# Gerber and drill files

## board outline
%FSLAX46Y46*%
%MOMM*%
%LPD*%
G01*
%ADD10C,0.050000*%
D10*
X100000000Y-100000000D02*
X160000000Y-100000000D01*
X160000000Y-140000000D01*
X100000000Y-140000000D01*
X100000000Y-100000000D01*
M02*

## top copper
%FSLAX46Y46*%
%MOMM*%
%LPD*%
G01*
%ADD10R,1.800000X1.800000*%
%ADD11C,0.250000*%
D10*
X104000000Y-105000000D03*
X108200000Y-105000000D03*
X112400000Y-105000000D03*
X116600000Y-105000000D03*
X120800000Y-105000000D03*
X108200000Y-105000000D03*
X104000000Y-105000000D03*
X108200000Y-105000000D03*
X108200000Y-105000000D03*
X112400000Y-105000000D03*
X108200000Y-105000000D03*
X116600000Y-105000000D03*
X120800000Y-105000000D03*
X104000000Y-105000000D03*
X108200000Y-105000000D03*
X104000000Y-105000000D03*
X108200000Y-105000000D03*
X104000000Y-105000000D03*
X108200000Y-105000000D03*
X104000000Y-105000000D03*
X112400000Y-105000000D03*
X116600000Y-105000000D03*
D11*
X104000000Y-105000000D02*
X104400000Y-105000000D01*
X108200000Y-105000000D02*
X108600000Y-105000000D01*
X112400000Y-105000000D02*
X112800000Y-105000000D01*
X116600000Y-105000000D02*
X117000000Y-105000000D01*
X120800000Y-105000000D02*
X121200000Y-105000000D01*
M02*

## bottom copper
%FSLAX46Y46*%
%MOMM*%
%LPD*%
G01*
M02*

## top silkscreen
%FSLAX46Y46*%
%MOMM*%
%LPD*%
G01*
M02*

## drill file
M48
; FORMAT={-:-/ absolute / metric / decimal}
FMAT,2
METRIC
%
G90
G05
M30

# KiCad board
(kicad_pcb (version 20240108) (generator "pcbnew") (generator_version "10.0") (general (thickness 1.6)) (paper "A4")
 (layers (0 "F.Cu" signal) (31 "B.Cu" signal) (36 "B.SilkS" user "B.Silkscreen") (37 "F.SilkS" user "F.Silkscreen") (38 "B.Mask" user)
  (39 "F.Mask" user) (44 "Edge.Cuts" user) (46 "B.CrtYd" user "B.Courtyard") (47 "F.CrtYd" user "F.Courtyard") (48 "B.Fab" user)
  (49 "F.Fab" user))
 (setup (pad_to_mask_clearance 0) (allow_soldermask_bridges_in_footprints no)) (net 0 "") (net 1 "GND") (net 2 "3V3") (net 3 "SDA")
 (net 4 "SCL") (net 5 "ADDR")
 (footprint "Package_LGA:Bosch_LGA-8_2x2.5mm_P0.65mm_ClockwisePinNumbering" (layer "F.Cu") (at 100 100)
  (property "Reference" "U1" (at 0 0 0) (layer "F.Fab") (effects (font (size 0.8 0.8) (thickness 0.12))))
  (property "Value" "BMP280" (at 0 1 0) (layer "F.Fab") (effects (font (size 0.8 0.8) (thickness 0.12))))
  (pad "1" smd rect (at 4.000 5.000) (size 1.8 1.8) (layers "F.Cu" "F.Paste" "F.Mask") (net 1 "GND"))
  (pad "2" smd rect (at 8.200 5.000) (size 1.8 1.8) (layers "F.Cu" "F.Paste" "F.Mask") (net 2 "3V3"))
  (pad "3" smd rect (at 12.400 5.000) (size 1.8 1.8) (layers "F.Cu" "F.Paste" "F.Mask") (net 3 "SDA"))
  (pad "4" smd rect (at 16.600 5.000) (size 1.8 1.8) (layers "F.Cu" "F.Paste" "F.Mask") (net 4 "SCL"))
  (pad "5" smd rect (at 20.800 5.000) (size 1.8 1.8) (layers "F.Cu" "F.Paste" "F.Mask") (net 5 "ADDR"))
  (pad "6" smd rect (at 8.200 5.000) (size 1.8 1.8) (layers "F.Cu" "F.Paste" "F.Mask") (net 2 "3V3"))
  (pad "7" smd rect (at 4.000 5.000) (size 1.8 1.8) (layers "F.Cu" "F.Paste" "F.Mask") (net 1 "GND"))
  (pad "8" smd rect (at 8.200 5.000) (size 1.8 1.8) (layers "F.Cu" "F.Paste" "F.Mask") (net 2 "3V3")))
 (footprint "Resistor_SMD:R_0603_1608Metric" (layer "F.Cu") (at 100 100)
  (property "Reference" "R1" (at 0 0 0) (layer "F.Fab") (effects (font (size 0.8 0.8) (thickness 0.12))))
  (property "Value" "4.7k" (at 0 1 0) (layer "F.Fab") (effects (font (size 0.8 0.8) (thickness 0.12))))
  (pad "1" smd rect (at 8.200 5.000) (size 1.8 1.8) (layers "F.Cu" "F.Paste" "F.Mask") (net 2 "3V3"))
  (pad "2" smd rect (at 12.400 5.000) (size 1.8 1.8) (layers "F.Cu" "F.Paste" "F.Mask") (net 3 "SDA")))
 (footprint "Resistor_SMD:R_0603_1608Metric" (layer "F.Cu") (at 100 100)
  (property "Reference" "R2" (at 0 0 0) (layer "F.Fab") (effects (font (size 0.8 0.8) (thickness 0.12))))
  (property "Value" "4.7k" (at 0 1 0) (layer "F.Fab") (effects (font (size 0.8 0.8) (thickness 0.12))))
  (pad "1" smd rect (at 8.200 5.000) (size 1.8 1.8) (layers "F.Cu" "F.Paste" "F.Mask") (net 2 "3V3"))
  (pad "2" smd rect (at 16.600 5.000) (size 1.8 1.8) (layers "F.Cu" "F.Paste" "F.Mask") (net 4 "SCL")))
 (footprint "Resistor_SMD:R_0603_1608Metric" (layer "F.Cu") (at 100 100)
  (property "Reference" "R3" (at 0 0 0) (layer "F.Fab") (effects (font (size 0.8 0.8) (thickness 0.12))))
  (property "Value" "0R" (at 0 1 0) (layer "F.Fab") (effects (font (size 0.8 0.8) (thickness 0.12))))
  (pad "1" smd rect (at 20.800 5.000) (size 1.8 1.8) (layers "F.Cu" "F.Paste" "F.Mask") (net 5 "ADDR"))
  (pad "2" smd rect (at 4.000 5.000) (size 1.8 1.8) (layers "F.Cu" "F.Paste" "F.Mask") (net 1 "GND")))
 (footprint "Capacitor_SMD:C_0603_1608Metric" (layer "F.Cu") (at 100 100)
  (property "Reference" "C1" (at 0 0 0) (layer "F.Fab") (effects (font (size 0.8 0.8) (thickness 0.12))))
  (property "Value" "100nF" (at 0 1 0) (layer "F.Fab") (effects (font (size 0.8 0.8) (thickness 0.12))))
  (pad "1" smd rect (at 8.200 5.000) (size 1.8 1.8) (layers "F.Cu" "F.Paste" "F.Mask") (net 2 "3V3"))
  (pad "2" smd rect (at 4.000 5.000) (size 1.8 1.8) (layers "F.Cu" "F.Paste" "F.Mask") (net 1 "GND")))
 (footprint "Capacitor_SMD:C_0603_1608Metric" (layer "F.Cu") (at 100 100)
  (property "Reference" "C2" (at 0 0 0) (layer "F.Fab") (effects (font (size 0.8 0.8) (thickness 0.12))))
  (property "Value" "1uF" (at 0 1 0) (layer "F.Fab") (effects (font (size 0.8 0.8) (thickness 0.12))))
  (pad "1" smd rect (at 8.200 5.000) (size 1.8 1.8) (layers "F.Cu" "F.Paste" "F.Mask") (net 2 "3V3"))
  (pad "2" smd rect (at 4.000 5.000) (size 1.8 1.8) (layers "F.Cu" "F.Paste" "F.Mask") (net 1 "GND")))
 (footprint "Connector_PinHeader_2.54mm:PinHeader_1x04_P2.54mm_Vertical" (layer "F.Cu") (at 100 100)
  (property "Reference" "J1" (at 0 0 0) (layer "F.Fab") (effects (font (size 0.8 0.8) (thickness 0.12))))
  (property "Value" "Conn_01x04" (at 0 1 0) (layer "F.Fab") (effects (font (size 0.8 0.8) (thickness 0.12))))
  (pad "1" smd rect (at 8.200 5.000) (size 1.8 1.8) (layers "F.Cu" "F.Paste" "F.Mask") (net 2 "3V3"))
  (pad "2" smd rect (at 4.000 5.000) (size 1.8 1.8) (layers "F.Cu" "F.Paste" "F.Mask") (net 1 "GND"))
  (pad "3" smd rect (at 12.400 5.000) (size 1.8 1.8) (layers "F.Cu" "F.Paste" "F.Mask") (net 3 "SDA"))
  (pad "4" smd rect (at 16.600 5.000) (size 1.8 1.8) (layers "F.Cu" "F.Paste" "F.Mask") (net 4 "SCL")))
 (gr_rect (start 100 100) (end 160 140) (stroke (width 0.05) (type default)) (fill none) (layer "Edge.Cuts"))
 (segment (start 104.000 105.000) (end 104.400 105.000) (width 0.25) (layer "F.Cu") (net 1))
 (segment (start 108.200 105.000) (end 108.600 105.000) (width 0.25) (layer "F.Cu") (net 2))
 (segment (start 112.400 105.000) (end 112.800 105.000) (width 0.25) (layer "F.Cu") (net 3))
 (segment (start 116.600 105.000) (end 117.000 105.000) (width 0.25) (layer "F.Cu") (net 4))
 (segment (start 120.800 105.000) (end 121.200 105.000) (width 0.25) (layer "F.Cu") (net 5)))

